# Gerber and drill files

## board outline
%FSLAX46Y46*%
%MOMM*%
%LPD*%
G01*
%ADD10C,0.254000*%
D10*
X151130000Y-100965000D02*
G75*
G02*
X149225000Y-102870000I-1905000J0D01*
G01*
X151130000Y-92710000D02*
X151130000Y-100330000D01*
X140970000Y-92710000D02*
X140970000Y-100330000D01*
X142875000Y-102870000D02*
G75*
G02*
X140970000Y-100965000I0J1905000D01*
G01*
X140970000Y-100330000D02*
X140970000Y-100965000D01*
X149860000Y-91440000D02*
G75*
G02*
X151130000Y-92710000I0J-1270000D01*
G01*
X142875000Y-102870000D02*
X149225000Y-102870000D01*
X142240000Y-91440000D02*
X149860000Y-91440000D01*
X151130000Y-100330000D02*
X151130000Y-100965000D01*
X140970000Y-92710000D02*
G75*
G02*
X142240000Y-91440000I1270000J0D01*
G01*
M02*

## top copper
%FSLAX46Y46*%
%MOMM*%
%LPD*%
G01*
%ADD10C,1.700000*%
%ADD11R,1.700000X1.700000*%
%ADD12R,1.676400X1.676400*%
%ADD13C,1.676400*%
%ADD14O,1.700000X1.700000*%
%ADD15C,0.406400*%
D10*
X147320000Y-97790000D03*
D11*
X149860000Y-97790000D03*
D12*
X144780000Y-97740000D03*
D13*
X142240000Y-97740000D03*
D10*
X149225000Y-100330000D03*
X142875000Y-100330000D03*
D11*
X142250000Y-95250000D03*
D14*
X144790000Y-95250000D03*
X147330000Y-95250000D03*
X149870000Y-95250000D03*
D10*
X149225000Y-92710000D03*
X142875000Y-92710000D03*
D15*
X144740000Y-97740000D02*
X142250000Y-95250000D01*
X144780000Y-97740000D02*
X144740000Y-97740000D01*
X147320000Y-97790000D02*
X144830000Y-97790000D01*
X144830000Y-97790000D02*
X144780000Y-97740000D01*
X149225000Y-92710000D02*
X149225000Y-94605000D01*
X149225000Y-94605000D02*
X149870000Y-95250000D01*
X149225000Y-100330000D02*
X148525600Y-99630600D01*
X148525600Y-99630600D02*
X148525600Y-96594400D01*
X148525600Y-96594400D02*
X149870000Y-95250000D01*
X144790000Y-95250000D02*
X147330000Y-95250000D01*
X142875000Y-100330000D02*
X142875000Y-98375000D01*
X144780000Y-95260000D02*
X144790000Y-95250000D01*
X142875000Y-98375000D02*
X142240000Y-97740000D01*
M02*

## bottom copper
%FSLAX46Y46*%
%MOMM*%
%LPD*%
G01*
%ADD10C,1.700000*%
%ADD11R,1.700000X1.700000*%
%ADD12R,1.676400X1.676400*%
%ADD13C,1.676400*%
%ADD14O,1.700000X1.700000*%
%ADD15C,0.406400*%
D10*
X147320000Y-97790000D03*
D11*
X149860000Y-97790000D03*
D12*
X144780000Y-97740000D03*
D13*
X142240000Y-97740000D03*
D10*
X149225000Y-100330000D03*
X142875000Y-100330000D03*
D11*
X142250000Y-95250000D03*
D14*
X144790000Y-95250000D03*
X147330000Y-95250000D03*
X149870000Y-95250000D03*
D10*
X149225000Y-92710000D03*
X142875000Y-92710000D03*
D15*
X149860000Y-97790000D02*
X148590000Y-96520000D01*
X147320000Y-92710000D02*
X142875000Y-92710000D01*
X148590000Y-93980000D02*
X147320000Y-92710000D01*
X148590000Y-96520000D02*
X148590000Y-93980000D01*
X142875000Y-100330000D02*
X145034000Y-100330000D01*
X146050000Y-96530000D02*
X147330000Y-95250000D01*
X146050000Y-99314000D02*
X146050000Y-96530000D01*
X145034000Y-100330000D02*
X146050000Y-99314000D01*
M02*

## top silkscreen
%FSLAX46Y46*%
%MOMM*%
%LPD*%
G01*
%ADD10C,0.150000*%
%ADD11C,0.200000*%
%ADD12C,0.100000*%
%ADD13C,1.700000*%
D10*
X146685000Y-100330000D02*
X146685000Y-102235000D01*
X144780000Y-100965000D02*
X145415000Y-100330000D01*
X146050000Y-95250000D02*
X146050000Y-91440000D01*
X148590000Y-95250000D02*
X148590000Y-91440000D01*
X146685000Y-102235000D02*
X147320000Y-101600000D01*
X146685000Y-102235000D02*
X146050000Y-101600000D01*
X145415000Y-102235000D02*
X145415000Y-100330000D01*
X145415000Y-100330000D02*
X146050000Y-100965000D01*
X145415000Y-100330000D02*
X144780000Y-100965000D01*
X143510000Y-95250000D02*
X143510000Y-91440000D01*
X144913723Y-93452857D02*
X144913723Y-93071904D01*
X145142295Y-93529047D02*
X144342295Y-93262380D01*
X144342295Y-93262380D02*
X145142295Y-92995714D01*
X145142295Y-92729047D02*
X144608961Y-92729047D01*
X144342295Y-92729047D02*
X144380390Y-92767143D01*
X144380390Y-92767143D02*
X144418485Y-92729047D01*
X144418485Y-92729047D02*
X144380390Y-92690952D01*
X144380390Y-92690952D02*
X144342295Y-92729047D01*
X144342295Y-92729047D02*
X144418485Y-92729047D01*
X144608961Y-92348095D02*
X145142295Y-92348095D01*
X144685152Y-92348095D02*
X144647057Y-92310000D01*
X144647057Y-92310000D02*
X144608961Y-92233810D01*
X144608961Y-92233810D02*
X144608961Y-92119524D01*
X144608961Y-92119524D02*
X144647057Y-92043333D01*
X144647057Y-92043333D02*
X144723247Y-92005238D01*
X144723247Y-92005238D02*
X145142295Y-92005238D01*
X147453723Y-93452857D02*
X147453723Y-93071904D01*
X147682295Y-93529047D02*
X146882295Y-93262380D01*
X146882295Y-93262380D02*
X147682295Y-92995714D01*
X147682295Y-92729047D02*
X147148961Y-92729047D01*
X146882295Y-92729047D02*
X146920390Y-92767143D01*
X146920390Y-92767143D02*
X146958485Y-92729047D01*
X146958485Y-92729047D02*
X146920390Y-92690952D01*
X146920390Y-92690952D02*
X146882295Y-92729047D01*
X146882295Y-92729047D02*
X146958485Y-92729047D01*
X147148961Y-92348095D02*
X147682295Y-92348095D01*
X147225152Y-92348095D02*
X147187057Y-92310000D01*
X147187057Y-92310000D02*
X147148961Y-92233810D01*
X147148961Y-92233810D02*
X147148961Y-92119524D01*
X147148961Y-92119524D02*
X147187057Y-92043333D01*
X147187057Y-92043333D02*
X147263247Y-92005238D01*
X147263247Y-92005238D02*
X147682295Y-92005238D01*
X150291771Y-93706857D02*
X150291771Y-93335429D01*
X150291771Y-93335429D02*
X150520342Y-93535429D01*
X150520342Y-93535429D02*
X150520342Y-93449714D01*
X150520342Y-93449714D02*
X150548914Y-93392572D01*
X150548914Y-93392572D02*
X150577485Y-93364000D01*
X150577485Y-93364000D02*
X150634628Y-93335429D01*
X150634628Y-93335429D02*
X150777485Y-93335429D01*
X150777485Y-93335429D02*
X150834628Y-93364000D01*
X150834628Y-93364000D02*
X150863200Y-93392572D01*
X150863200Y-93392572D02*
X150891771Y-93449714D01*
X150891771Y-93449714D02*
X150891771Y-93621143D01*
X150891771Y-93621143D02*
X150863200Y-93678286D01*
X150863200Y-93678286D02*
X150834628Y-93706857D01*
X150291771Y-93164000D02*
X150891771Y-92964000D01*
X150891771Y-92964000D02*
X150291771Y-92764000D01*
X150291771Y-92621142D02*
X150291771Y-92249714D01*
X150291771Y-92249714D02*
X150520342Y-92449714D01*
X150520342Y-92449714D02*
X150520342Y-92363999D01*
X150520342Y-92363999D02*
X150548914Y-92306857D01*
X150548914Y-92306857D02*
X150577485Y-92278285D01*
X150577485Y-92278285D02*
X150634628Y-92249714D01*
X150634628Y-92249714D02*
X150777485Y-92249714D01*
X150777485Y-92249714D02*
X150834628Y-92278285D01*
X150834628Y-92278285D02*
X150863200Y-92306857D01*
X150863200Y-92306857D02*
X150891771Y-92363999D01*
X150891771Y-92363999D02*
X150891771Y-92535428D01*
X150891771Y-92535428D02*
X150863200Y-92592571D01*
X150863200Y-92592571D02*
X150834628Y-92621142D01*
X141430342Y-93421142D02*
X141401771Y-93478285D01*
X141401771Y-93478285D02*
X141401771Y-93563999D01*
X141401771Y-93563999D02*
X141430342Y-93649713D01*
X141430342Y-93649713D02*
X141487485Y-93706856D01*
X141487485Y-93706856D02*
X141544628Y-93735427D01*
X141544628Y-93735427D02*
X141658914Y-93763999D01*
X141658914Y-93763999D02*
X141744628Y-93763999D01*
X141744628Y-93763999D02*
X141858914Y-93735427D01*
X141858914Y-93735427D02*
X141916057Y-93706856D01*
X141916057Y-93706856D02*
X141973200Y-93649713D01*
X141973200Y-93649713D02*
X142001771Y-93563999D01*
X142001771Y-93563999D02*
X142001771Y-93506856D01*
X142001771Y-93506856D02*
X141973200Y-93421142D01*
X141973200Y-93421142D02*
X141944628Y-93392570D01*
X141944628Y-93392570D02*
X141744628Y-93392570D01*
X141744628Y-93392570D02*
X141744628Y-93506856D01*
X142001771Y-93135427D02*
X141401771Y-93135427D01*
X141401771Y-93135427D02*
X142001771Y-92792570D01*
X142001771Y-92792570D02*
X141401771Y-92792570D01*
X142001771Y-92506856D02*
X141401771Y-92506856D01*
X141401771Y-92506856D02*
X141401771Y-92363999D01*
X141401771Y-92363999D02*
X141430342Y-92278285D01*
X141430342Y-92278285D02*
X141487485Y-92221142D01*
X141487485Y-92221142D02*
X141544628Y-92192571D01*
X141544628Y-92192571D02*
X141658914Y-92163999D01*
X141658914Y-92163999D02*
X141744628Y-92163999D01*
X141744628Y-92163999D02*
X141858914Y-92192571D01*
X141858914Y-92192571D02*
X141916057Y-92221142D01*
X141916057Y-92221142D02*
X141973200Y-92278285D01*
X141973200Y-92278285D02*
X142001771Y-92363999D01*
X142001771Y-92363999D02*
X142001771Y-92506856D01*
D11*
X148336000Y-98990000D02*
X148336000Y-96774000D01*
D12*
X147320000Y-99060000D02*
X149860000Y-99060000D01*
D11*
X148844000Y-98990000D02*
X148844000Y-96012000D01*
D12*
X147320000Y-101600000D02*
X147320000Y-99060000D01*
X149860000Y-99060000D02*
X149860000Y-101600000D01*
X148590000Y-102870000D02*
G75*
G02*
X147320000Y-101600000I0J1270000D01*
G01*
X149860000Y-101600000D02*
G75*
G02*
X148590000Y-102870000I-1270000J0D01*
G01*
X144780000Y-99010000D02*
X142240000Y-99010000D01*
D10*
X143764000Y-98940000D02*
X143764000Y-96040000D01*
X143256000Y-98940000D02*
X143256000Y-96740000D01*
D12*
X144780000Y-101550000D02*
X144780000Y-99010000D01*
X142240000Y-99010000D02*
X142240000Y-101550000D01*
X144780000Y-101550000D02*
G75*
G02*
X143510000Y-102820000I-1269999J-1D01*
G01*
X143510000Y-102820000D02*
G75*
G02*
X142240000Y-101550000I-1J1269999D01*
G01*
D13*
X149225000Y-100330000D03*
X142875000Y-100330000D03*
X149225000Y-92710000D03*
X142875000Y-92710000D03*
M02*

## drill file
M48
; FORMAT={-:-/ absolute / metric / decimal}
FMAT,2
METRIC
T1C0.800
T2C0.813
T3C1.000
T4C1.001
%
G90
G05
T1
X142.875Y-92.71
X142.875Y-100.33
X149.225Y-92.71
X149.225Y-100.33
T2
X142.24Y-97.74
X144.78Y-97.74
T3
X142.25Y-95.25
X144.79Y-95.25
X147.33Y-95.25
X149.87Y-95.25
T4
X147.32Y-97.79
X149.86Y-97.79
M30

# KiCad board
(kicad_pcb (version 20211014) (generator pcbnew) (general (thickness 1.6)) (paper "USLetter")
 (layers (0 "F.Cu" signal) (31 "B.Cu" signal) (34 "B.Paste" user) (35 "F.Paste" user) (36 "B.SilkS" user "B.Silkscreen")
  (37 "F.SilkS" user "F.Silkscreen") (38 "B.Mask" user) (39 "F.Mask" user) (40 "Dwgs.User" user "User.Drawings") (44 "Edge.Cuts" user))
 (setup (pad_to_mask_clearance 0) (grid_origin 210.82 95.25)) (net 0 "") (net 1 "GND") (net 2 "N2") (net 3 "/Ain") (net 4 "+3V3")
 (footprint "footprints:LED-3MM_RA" (layer "F.Cu") (at 147.32 97.79)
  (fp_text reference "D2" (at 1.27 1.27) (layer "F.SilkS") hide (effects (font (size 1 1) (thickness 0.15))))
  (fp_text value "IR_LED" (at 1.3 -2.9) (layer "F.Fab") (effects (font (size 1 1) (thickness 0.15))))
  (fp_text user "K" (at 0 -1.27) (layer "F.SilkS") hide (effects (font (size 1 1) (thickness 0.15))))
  (fp_line (start 1.016 1.2) (end 1.016 -1.016) (layer "F.SilkS") (width 0.2))
  (fp_line (start 0 1.27) (end 2.54 1.27) (layer "F.SilkS") (width 0.1))
  (fp_line (start 1.524 1.2) (end 1.524 -1.778) (layer "F.SilkS") (width 0.2))
  (fp_line (start 0 3.81) (end 0 1.27) (layer "F.SilkS") (width 0.1))
  (fp_line (start 2.54 1.27) (end 2.54 3.81) (layer "F.SilkS") (width 0.1))
  (fp_arc (start 1.27 5.08) (mid 0.371974 4.708026) (end 0 3.81) (layer "F.SilkS") (width 0.1))
  (fp_arc (start 2.54 3.81) (mid 2.168026 4.708026) (end 1.27 5.08) (layer "F.SilkS") (width 0.1))
  (pad "1" thru_hole circle (at 0 0 90) (size 1.7 1.7) (drill 1.00076) (layers *.Cu *.Mask) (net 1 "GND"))
  (pad "2" thru_hole rect (at 2.54 0) (size 1.7 1.7) (drill 1.00076) (layers *.Cu *.Mask) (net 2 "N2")))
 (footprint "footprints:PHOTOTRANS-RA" (layer "F.Cu") (at 143.51 97.74)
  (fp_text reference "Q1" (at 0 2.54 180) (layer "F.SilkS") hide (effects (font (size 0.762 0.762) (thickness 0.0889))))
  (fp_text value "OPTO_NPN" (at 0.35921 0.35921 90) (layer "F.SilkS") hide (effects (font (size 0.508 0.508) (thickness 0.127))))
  (fp_line (start 1.27 1.27) (end -1.27 1.27) (layer "F.SilkS") (width 0.1))
  (fp_line (start 0.254 1.2) (end 0.254 -1.7) (layer "F.SilkS") (width 0.15))
  (fp_line (start -0.254 1.2) (end -0.254 -1) (layer "F.SilkS") (width 0.15))
  (fp_line (start 1.27 3.81) (end 1.27 1.27) (layer "F.SilkS") (width 0.1))
  (fp_line (start -1.27 1.27) (end -1.27 3.81) (layer "F.SilkS") (width 0.1))
  (fp_arc (start 1.27 3.81) (mid 0.898026 4.708026) (end 0 5.08) (layer "F.SilkS") (width 0.1))
  (fp_arc (start 0 5.08) (mid -0.898026 4.708026) (end -1.27 3.81) (layer "F.SilkS") (width 0.1))
  (pad "1" thru_hole rect (at 1.27 0) (size 1.6764 1.6764) (drill 0.8128) (layers *.Cu *.Mask) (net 1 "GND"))
  (pad "3" thru_hole circle (at -1.27 0) (size 1.6764 1.6764) (drill 0.8128) (layers *.Cu *.Mask) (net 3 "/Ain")))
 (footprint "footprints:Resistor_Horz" (layer "B.Cu") (at 146.05 100.33 180)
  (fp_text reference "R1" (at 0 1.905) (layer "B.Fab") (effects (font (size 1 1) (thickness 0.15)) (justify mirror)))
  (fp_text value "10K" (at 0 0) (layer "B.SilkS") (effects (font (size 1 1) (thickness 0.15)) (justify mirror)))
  (pad "1" thru_hole circle (at -3.175 0 180) (size 1.7 1.7) (drill 0.8) (layers *.Cu *.SilkS *.Mask) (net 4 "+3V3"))
  (pad "2" thru_hole circle (at 3.175 0 180) (size 1.7 1.7) (drill 0.8) (layers *.Cu *.SilkS *.Mask) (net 3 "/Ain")))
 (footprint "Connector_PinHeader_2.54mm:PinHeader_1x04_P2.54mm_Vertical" (layer "B.Cu") (at 142.25 95.25 -90)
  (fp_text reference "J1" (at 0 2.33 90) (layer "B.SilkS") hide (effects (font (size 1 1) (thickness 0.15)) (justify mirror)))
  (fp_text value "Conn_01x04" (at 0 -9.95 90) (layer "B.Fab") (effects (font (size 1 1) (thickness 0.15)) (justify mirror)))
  (pad "1" thru_hole rect (at 0 0 270) (size 1.7 1.7) (drill 1) (layers *.Cu *.Mask) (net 1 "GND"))
  (pad "2" thru_hole oval (at 0 -2.54 270) (size 1.7 1.7) (drill 1) (layers *.Cu *.Mask) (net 3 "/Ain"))
  (pad "3" thru_hole oval (at 0 -5.08 270) (size 1.7 1.7) (drill 1) (layers *.Cu *.Mask) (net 3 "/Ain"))
  (pad "4" thru_hole oval (at 0 -7.62 270) (size 1.7 1.7) (drill 1) (layers *.Cu *.Mask) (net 4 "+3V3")))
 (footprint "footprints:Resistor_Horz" (layer "B.Cu") (at 146.05 92.71 180)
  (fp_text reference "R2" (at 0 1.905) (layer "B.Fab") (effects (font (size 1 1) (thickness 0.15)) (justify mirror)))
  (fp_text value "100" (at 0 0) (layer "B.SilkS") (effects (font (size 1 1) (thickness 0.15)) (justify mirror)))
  (pad "1" thru_hole circle (at -3.175 0 180) (size 1.7 1.7) (drill 0.8) (layers *.Cu *.SilkS *.Mask) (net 4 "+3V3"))
  (pad "2" thru_hole circle (at 3.175 0 180) (size 1.7 1.7) (drill 0.8) (layers *.Cu *.SilkS *.Mask) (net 2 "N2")))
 (gr_line (start 146.685 100.33) (end 146.685 102.235) (layer "F.SilkS") (width 0.15))
 (gr_line (start 144.78 100.965) (end 145.415 100.33) (layer "F.SilkS") (width 0.15))
 (gr_line (start 146.05 95.25) (end 146.05 91.44) (layer "F.SilkS") (width 0.15))
 (gr_line (start 148.59 95.25) (end 148.59 91.44) (layer "F.SilkS") (width 0.15))
 (gr_line (start 146.685 102.235) (end 147.32 101.6) (layer "F.SilkS") (width 0.15))
 (gr_line (start 146.685 102.235) (end 146.05 101.6) (layer "F.SilkS") (width 0.15))
 (gr_line (start 145.415 102.235) (end 145.415 100.33) (layer "F.SilkS") (width 0.15))
 (gr_line (start 145.415 100.33) (end 146.05 100.965) (layer "F.SilkS") (width 0.15))
 (gr_line (start 145.415 100.33) (end 144.78 100.965) (layer "F.SilkS") (width 0.15))
 (gr_line (start 143.51 95.25) (end 143.51 91.44) (layer "F.SilkS") (width 0.15))
 (gr_arc (start 151.13 100.965) (mid 150.572038 102.312038) (end 149.225 102.87) (layer "Edge.Cuts") (width 0.254))
 (gr_line (start 151.13 92.71) (end 151.13 100.33) (layer "Edge.Cuts") (width 0.254))
 (gr_line (start 140.97 92.71) (end 140.97 100.33) (layer "Edge.Cuts") (width 0.254))
 (gr_arc (start 142.875 102.87) (mid 141.527962 102.312038) (end 140.97 100.965) (layer "Edge.Cuts") (width 0.254))
 (gr_line (start 140.97 100.33) (end 140.97 100.965) (layer "Edge.Cuts") (width 0.254))
 (gr_arc (start 149.86 91.44) (mid 150.758026 91.811974) (end 151.13 92.71) (layer "Edge.Cuts") (width 0.254))
 (gr_line (start 142.875 102.87) (end 149.225 102.87) (layer "Edge.Cuts") (width 0.254))
 (gr_line (start 142.24 91.44) (end 149.86 91.44) (layer "Edge.Cuts") (width 0.254))
 (gr_line (start 151.13 100.33) (end 151.13 100.965) (layer "Edge.Cuts") (width 0.254))
 (gr_arc (start 140.97 92.71) (mid 141.341974 91.811974) (end 142.24 91.44) (layer "Edge.Cuts") (width 0.254))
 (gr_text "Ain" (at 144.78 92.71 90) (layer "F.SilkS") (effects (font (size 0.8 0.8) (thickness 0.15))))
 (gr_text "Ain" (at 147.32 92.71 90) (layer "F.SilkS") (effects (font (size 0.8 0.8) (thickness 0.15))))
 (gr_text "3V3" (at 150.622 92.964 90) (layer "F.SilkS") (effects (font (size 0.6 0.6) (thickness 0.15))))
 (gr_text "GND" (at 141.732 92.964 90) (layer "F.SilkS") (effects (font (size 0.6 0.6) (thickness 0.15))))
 (segment (start 144.74 97.74) (end 142.25 95.25) (width 0.4064) (layer "F.Cu") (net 1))
 (segment (start 144.78 97.74) (end 144.74 97.74) (width 0.4064) (layer "F.Cu") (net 1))
 (segment (start 147.32 97.79) (end 144.83 97.79) (width 0.4064) (layer "F.Cu") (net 1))
 (segment (start 144.83 97.79) (end 144.78 97.74) (width 0.4064) (layer "F.Cu") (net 1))
 (segment (start 149.86 97.79) (end 148.59 96.52) (width 0.4064) (layer "B.Cu") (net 2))
 (segment (start 147.32 92.71) (end 142.875 92.71) (width 0.4064) (layer "B.Cu") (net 2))
 (segment (start 148.59 93.98) (end 147.32 92.71) (width 0.4064) (layer "B.Cu") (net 2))
 (segment (start 148.59 96.52) (end 148.59 93.98) (width 0.4064) (layer "B.Cu") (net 2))
 (segment (start 149.225 92.71) (end 149.225 94.605) (width 0.4064) (layer "F.Cu") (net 4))
 (segment (start 149.225 94.605) (end 149.87 95.25) (width 0.4064) (layer "F.Cu") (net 4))
 (segment (start 149.225 100.33) (end 148.5256 99.6306) (width 0.4064) (layer "F.Cu") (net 4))
 (segment (start 148.5256 99.6306) (end 148.5256 96.5944) (width 0.4064) (layer "F.Cu") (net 4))
 (segment (start 148.5256 96.5944) (end 149.87 95.25) (width 0.4064) (layer "F.Cu") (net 4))
 (segment (start 144.79 95.25) (end 147.33 95.25) (width 0.4064) (layer "F.Cu") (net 3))
 (segment (start 142.875 100.33) (end 142.875 98.375) (width 0.4064) (layer "F.Cu") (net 3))
 (segment (start 144.78 95.26) (end 144.79 95.25) (width 0.4064) (layer "F.Cu") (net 3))
 (segment (start 142.875 98.375) (end 142.24 97.74) (width 0.4064) (layer "F.Cu") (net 3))
 (segment (start 142.875 100.33) (end 145.034 100.33) (width 0.4064) (layer "B.Cu") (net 3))
 (segment (start 146.05 96.53) (end 147.33 95.25) (width 0.4064) (layer "B.Cu") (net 3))
 (segment (start 146.05 99.314) (end 146.05 96.53) (width 0.4064) (layer "B.Cu") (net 3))
 (segment (start 145.034 100.33) (end 146.05 99.314) (width 0.4064) (layer "B.Cu") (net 3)))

